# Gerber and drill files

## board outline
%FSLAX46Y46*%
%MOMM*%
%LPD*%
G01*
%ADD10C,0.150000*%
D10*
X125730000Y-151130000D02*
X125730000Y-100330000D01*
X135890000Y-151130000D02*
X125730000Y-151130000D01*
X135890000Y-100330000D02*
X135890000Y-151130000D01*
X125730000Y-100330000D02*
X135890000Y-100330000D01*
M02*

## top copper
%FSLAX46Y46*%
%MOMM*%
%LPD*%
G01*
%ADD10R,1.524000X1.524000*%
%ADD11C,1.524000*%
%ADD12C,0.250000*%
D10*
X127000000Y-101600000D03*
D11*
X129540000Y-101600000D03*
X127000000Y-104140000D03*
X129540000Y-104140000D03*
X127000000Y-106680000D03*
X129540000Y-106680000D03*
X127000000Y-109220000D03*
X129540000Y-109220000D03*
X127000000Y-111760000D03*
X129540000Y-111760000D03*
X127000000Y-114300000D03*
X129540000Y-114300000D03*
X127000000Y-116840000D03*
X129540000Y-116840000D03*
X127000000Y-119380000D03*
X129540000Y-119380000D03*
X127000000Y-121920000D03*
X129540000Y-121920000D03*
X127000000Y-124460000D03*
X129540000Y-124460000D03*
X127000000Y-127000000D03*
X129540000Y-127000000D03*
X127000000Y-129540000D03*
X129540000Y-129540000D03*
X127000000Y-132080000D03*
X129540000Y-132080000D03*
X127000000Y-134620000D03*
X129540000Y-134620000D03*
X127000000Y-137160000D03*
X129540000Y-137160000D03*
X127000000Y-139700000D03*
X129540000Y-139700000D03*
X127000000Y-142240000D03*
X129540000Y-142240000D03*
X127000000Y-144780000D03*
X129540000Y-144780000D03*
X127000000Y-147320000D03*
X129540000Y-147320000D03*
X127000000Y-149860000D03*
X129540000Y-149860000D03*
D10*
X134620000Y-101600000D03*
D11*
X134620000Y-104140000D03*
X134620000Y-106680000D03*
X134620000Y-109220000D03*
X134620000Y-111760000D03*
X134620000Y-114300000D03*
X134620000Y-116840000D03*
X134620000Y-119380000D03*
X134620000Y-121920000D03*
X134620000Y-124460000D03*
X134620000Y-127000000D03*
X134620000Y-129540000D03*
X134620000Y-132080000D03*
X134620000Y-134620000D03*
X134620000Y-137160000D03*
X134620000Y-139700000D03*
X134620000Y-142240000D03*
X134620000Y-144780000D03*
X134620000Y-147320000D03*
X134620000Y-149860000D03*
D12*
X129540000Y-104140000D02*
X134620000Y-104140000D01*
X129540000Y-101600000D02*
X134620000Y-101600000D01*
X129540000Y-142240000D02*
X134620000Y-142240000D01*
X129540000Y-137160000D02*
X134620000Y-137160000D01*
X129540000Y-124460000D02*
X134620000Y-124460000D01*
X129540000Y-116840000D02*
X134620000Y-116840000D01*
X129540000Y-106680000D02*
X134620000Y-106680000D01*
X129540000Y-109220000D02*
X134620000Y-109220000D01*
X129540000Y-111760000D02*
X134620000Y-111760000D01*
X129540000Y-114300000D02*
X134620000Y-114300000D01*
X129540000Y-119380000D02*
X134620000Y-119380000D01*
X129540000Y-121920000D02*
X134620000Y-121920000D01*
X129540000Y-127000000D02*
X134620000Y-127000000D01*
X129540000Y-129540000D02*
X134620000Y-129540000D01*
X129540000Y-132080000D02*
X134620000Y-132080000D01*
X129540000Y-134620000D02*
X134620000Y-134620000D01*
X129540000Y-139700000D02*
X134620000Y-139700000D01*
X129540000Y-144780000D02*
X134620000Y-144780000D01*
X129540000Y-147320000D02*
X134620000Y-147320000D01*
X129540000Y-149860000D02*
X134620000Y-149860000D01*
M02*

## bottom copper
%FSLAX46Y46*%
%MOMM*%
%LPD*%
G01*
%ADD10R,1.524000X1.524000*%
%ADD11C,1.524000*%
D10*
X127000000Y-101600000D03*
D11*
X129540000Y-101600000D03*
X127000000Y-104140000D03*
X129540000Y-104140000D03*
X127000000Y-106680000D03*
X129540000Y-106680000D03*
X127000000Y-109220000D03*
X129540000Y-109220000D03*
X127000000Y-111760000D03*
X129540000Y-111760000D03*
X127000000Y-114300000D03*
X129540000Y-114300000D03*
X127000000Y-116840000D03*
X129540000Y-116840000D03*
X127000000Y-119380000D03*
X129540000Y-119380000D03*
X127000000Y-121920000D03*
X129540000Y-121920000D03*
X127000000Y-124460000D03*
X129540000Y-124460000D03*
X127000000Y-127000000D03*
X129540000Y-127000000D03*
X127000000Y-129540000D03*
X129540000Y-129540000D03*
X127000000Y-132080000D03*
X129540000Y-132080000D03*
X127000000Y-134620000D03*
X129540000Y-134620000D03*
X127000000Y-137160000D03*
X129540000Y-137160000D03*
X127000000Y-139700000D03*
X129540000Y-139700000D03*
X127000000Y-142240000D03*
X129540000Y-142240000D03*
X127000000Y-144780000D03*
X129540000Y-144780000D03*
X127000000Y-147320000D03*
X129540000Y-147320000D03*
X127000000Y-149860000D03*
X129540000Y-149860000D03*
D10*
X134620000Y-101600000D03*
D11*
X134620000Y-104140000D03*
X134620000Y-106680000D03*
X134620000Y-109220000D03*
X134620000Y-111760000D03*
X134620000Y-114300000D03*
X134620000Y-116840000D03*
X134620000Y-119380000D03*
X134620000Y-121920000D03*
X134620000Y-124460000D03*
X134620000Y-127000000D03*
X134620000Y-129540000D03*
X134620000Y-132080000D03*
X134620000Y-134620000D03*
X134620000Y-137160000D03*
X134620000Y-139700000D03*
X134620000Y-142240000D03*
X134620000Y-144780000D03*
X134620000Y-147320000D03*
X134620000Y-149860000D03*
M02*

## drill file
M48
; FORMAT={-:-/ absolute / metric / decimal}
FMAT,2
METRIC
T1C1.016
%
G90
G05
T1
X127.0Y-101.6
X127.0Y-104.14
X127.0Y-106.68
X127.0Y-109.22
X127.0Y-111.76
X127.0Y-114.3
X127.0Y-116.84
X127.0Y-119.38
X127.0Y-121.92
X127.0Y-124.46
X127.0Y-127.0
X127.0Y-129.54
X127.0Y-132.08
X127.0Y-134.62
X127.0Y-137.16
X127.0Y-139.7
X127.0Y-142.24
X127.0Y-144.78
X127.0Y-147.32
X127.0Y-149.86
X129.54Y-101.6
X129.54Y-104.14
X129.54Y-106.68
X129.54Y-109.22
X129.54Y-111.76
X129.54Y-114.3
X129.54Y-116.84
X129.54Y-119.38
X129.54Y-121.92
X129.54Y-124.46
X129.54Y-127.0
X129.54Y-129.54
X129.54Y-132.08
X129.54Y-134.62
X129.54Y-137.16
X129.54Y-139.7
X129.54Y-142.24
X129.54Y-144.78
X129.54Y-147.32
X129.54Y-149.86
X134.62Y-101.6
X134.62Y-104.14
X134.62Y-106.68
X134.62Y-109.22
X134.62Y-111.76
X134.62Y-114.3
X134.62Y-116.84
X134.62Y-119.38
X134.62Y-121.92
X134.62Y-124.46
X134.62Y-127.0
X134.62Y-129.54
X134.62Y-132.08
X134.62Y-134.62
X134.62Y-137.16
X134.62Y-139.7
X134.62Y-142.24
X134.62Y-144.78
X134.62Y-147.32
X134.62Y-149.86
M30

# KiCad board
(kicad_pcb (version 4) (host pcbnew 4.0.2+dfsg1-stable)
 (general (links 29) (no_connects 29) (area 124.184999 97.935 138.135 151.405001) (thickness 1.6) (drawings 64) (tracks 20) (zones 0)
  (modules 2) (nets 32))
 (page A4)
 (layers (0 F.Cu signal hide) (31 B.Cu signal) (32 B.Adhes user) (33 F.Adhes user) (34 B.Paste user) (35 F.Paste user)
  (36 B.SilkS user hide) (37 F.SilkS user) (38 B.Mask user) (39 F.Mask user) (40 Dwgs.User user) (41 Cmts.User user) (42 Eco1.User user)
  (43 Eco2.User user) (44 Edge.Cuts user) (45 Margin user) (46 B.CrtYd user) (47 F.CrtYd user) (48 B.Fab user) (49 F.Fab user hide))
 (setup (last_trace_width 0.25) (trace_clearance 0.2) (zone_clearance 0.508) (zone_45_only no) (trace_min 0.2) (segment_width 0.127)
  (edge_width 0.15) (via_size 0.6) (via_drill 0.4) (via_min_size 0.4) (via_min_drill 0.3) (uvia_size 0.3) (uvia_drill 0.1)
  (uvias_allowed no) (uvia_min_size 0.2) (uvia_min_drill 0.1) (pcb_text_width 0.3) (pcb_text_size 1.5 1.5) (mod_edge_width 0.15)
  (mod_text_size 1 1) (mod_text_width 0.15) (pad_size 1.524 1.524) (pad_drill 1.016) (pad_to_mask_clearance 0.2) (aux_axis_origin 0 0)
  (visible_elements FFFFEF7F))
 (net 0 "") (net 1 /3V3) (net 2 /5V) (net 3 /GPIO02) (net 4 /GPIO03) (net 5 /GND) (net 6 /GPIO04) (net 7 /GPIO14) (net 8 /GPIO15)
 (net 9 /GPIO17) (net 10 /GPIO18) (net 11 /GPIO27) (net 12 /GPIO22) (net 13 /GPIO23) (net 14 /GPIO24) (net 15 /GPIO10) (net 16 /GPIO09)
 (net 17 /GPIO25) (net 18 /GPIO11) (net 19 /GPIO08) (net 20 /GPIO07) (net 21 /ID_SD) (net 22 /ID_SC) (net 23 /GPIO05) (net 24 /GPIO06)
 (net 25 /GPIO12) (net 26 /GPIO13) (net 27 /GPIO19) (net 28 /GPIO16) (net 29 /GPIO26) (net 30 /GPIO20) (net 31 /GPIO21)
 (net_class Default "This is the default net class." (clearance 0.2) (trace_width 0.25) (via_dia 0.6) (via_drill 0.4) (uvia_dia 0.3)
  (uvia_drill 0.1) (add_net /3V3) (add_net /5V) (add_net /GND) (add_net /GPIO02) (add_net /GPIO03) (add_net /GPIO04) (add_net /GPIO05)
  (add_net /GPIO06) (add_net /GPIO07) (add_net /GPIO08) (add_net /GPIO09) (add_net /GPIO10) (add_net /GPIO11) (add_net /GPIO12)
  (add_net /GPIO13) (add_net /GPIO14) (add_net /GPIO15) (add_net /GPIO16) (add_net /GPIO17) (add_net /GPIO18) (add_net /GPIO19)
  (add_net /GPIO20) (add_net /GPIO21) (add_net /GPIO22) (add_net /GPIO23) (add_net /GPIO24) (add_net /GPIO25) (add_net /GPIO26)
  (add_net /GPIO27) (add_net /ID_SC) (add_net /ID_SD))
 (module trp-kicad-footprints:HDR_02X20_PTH (layer F.Cu) (at 127 101.6)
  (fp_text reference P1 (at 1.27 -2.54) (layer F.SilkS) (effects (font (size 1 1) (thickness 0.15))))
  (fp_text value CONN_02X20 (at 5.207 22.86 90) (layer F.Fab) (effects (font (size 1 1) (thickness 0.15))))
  (pad 1 thru_hole rect (at 0 0) (size 1.524 1.524) (drill 1.016) (layers *.Cu *.Mask F.SilkS) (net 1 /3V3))
  (pad 2 thru_hole circle (at 2.54 0) (size 1.524 1.524) (drill 1.016) (layers *.Cu *.Mask F.SilkS) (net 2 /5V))
  (pad 3 thru_hole circle (at 0 2.54) (size 1.524 1.524) (drill 1.016) (layers *.Cu *.Mask F.SilkS) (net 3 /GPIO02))
  (pad 4 thru_hole circle (at 2.54 2.54) (size 1.524 1.524) (drill 1.016) (layers *.Cu *.Mask F.SilkS) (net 2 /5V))
  (pad 5 thru_hole circle (at 0 5.08) (size 1.524 1.524) (drill 1.016) (layers *.Cu *.Mask F.SilkS) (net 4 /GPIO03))
  (pad 6 thru_hole circle (at 2.54 5.08) (size 1.524 1.524) (drill 1.016) (layers *.Cu *.Mask F.SilkS) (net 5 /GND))
  (pad 7 thru_hole circle (at 0 7.62) (size 1.524 1.524) (drill 1.016) (layers *.Cu *.Mask F.SilkS) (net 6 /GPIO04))
  (pad 8 thru_hole circle (at 2.54 7.62) (size 1.524 1.524) (drill 1.016) (layers *.Cu *.Mask F.SilkS) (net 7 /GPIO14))
  (pad 9 thru_hole circle (at 0 10.16) (size 1.524 1.524) (drill 1.016) (layers *.Cu *.Mask F.SilkS) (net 5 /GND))
  (pad 10 thru_hole circle (at 2.54 10.16) (size 1.524 1.524) (drill 1.016) (layers *.Cu *.Mask F.SilkS) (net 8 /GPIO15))
  (pad 11 thru_hole circle (at 0 12.7) (size 1.524 1.524) (drill 1.016) (layers *.Cu *.Mask F.SilkS) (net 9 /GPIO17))
  (pad 12 thru_hole circle (at 2.54 12.7) (size 1.524 1.524) (drill 1.016) (layers *.Cu *.Mask F.SilkS) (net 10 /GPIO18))
  (pad 13 thru_hole circle (at 0 15.24) (size 1.524 1.524) (drill 1.016) (layers *.Cu *.Mask F.SilkS) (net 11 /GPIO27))
  (pad 14 thru_hole circle (at 2.54 15.24) (size 1.524 1.524) (drill 1.016) (layers *.Cu *.Mask F.SilkS) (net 5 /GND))
  (pad 15 thru_hole circle (at 0 17.78) (size 1.524 1.524) (drill 1.016) (layers *.Cu *.Mask F.SilkS) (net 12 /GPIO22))
  (pad 16 thru_hole circle (at 2.54 17.78) (size 1.524 1.524) (drill 1.016) (layers *.Cu *.Mask F.SilkS) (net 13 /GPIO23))
  (pad 17 thru_hole circle (at 0 20.32) (size 1.524 1.524) (drill 1.016) (layers *.Cu *.Mask F.SilkS) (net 1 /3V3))
  (pad 18 thru_hole circle (at 2.54 20.32) (size 1.524 1.524) (drill 1.016) (layers *.Cu *.Mask F.SilkS) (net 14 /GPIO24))
  (pad 19 thru_hole circle (at 0 22.86) (size 1.524 1.524) (drill 1.016) (layers *.Cu *.Mask F.SilkS) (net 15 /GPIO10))
  (pad 20 thru_hole circle (at 2.54 22.86) (size 1.524 1.524) (drill 1.016) (layers *.Cu *.Mask F.SilkS) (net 5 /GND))
  (pad 21 thru_hole circle (at 0 25.4) (size 1.524 1.524) (drill 1.016) (layers *.Cu *.Mask F.SilkS) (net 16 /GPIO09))
  (pad 22 thru_hole circle (at 2.54 25.4) (size 1.524 1.524) (drill 1.016) (layers *.Cu *.Mask F.SilkS) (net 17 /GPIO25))
  (pad 23 thru_hole circle (at 0 27.94) (size 1.524 1.524) (drill 1.016) (layers *.Cu *.Mask F.SilkS) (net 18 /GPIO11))
  (pad 24 thru_hole circle (at 2.54 27.94) (size 1.524 1.524) (drill 1.016) (layers *.Cu *.Mask F.SilkS) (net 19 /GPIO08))
  (pad 25 thru_hole circle (at 0 30.48) (size 1.524 1.524) (drill 1.016) (layers *.Cu *.Mask F.SilkS) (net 5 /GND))
  (pad 26 thru_hole circle (at 2.54 30.48) (size 1.524 1.524) (drill 1.016) (layers *.Cu *.Mask F.SilkS) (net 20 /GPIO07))
  (pad 27 thru_hole circle (at 0 33.02) (size 1.524 1.524) (drill 1.016) (layers *.Cu *.Mask F.SilkS) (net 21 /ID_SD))
  (pad 28 thru_hole circle (at 2.54 33.02) (size 1.524 1.524) (drill 1.016) (layers *.Cu *.Mask F.SilkS) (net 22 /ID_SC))
  (pad 29 thru_hole circle (at 0 35.56) (size 1.524 1.524) (drill 1.016) (layers *.Cu *.Mask F.SilkS) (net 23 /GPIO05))
  (pad 30 thru_hole circle (at 2.54 35.56) (size 1.524 1.524) (drill 1.016) (layers *.Cu *.Mask F.SilkS) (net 5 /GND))
  (pad 31 thru_hole circle (at 0 38.1) (size 1.524 1.524) (drill 1.016) (layers *.Cu *.Mask F.SilkS) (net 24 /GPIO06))
  (pad 32 thru_hole circle (at 2.54 38.1) (size 1.524 1.524) (drill 1.016) (layers *.Cu *.Mask F.SilkS) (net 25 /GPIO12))
  (pad 33 thru_hole circle (at 0 40.64) (size 1.524 1.524) (drill 1.016) (layers *.Cu *.Mask F.SilkS) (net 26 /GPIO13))
  (pad 34 thru_hole circle (at 2.54 40.64) (size 1.524 1.524) (drill 1.016) (layers *.Cu *.Mask F.SilkS) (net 5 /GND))
  (pad 35 thru_hole circle (at 0 43.18) (size 1.524 1.524) (drill 1.016) (layers *.Cu *.Mask F.SilkS) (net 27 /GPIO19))
  (pad 36 thru_hole circle (at 2.54 43.18) (size 1.524 1.524) (drill 1.016) (layers *.Cu *.Mask F.SilkS) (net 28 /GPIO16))
  (pad 37 thru_hole circle (at 0 45.72) (size 1.524 1.524) (drill 1.016) (layers *.Cu *.Mask F.SilkS) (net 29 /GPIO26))
  (pad 38 thru_hole circle (at 2.54 45.72) (size 1.524 1.524) (drill 1.016) (layers *.Cu *.Mask F.SilkS) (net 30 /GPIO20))
  (pad 39 thru_hole circle (at 0 48.26) (size 1.524 1.524) (drill 1.016) (layers *.Cu *.Mask F.SilkS) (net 5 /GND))
  (pad 40 thru_hole circle (at 2.54 48.26) (size 1.524 1.524) (drill 1.016) (layers *.Cu *.Mask F.SilkS) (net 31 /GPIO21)))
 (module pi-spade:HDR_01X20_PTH (layer F.Cu) (at 134.62 124.46)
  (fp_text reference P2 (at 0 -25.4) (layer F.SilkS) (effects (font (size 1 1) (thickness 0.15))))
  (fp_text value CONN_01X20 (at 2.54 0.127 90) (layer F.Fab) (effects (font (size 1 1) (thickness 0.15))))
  (pad 1 thru_hole rect (at 0 -22.86) (size 1.524 1.524) (drill 1.016) (layers *.Cu *.Mask F.SilkS) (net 2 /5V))
  (pad 2 thru_hole circle (at 0 -20.32) (size 1.524 1.524) (drill 1.016) (layers *.Cu *.Mask F.SilkS) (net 2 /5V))
  (pad 3 thru_hole circle (at 0 -17.78) (size 1.524 1.524) (drill 1.016) (layers *.Cu *.Mask F.SilkS) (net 5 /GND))
  (pad 4 thru_hole circle (at 0 -15.24) (size 1.524 1.524) (drill 1.016) (layers *.Cu *.Mask F.SilkS) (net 7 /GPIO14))
  (pad 5 thru_hole circle (at 0 -12.7) (size 1.524 1.524) (drill 1.016) (layers *.Cu *.Mask F.SilkS) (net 8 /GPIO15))
  (pad 6 thru_hole circle (at 0 -10.16) (size 1.524 1.524) (drill 1.016) (layers *.Cu *.Mask F.SilkS) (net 10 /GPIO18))
  (pad 7 thru_hole circle (at 0 -7.62) (size 1.524 1.524) (drill 1.016) (layers *.Cu *.Mask F.SilkS) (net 5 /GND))
  (pad 8 thru_hole circle (at 0 -5.08) (size 1.524 1.524) (drill 1.016) (layers *.Cu *.Mask F.SilkS) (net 13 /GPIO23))
  (pad 9 thru_hole circle (at 0 -2.54) (size 1.524 1.524) (drill 1.016) (layers *.Cu *.Mask F.SilkS) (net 14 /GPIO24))
  (pad 10 thru_hole circle (at 0 0) (size 1.524 1.524) (drill 1.016) (layers *.Cu *.Mask F.SilkS) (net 5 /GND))
  (pad 11 thru_hole circle (at 0 2.54) (size 1.524 1.524) (drill 1.016) (layers *.Cu *.Mask F.SilkS) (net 17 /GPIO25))
  (pad 12 thru_hole circle (at 0 5.08) (size 1.524 1.524) (drill 1.016) (layers *.Cu *.Mask F.SilkS) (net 19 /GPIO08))
  (pad 13 thru_hole circle (at 0 7.62) (size 1.524 1.524) (drill 1.016) (layers *.Cu *.Mask F.SilkS) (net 20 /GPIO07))
  (pad 14 thru_hole circle (at 0 10.16) (size 1.524 1.524) (drill 1.016) (layers *.Cu *.Mask F.SilkS) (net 22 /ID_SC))
  (pad 15 thru_hole circle (at 0 12.7) (size 1.524 1.524) (drill 1.016) (layers *.Cu *.Mask F.SilkS) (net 5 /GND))
  (pad 16 thru_hole circle (at 0 15.24) (size 1.524 1.524) (drill 1.016) (layers *.Cu *.Mask F.SilkS) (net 25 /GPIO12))
  (pad 17 thru_hole circle (at 0 17.78) (size 1.524 1.524) (drill 1.016) (layers *.Cu *.Mask F.SilkS) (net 5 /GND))
  (pad 18 thru_hole circle (at 0 20.32) (size 1.524 1.524) (drill 1.016) (layers *.Cu *.Mask F.SilkS) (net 28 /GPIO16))
  (pad 19 thru_hole circle (at 0 22.86) (size 1.524 1.524) (drill 1.016) (layers *.Cu *.Mask F.SilkS) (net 30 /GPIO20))
  (pad 20 thru_hole circle (at 0 25.4) (size 1.524 1.524) (drill 1.016) (layers *.Cu *.Mask F.SilkS) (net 31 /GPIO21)))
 (gr_line (start 125.73 151.13) (end 125.73 100.33) (layer Edge.Cuts) (width 0.15))
 (gr_line (start 135.89 151.13) (end 125.73 151.13) (layer Edge.Cuts) (width 0.15))
 (gr_line (start 135.89 100.33) (end 135.89 151.13) (layer Edge.Cuts) (width 0.15))
 (gr_line (start 125.73 100.33) (end 135.89 100.33) (layer Edge.Cuts) (width 0.15))
 (segment (start 129.54 104.14) (end 134.62 104.14) (width 0.25) (layer F.Cu) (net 2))
 (segment (start 129.54 101.6) (end 134.62 101.6) (width 0.25) (layer F.Cu) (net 2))
 (segment (start 129.54 142.24) (end 134.62 142.24) (width 0.25) (layer F.Cu) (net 5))
 (segment (start 129.54 137.16) (end 134.62 137.16) (width 0.25) (layer F.Cu) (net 5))
 (segment (start 129.54 124.46) (end 134.62 124.46) (width 0.25) (layer F.Cu) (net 5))
 (segment (start 129.54 116.84) (end 134.62 116.84) (width 0.25) (layer F.Cu) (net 5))
 (segment (start 129.54 106.68) (end 134.62 106.68) (width 0.25) (layer F.Cu) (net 5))
 (segment (start 129.54 109.22) (end 134.62 109.22) (width 0.25) (layer F.Cu) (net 7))
 (segment (start 129.54 111.76) (end 134.62 111.76) (width 0.25) (layer F.Cu) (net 8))
 (segment (start 129.54 114.3) (end 134.62 114.3) (width 0.25) (layer F.Cu) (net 10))
 (segment (start 129.54 119.38) (end 134.62 119.38) (width 0.25) (layer F.Cu) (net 13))
 (segment (start 129.54 121.92) (end 134.62 121.92) (width 0.25) (layer F.Cu) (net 14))
 (segment (start 129.54 127) (end 134.62 127) (width 0.25) (layer F.Cu) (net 17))
 (segment (start 129.54 129.54) (end 134.62 129.54) (width 0.25) (layer F.Cu) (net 19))
 (segment (start 129.54 132.08) (end 134.62 132.08) (width 0.25) (layer F.Cu) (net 20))
 (segment (start 129.54 134.62) (end 134.62 134.62) (width 0.25) (layer F.Cu) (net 22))
 (segment (start 129.54 139.7) (end 134.62 139.7) (width 0.25) (layer F.Cu) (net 25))
 (segment (start 129.54 144.78) (end 134.62 144.78) (width 0.25) (layer F.Cu) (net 28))
 (segment (start 129.54 147.32) (end 134.62 147.32) (width 0.25) (layer F.Cu) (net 30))
 (segment (start 129.54 149.86) (end 134.62 149.86) (width 0.25) (layer F.Cu) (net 31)))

